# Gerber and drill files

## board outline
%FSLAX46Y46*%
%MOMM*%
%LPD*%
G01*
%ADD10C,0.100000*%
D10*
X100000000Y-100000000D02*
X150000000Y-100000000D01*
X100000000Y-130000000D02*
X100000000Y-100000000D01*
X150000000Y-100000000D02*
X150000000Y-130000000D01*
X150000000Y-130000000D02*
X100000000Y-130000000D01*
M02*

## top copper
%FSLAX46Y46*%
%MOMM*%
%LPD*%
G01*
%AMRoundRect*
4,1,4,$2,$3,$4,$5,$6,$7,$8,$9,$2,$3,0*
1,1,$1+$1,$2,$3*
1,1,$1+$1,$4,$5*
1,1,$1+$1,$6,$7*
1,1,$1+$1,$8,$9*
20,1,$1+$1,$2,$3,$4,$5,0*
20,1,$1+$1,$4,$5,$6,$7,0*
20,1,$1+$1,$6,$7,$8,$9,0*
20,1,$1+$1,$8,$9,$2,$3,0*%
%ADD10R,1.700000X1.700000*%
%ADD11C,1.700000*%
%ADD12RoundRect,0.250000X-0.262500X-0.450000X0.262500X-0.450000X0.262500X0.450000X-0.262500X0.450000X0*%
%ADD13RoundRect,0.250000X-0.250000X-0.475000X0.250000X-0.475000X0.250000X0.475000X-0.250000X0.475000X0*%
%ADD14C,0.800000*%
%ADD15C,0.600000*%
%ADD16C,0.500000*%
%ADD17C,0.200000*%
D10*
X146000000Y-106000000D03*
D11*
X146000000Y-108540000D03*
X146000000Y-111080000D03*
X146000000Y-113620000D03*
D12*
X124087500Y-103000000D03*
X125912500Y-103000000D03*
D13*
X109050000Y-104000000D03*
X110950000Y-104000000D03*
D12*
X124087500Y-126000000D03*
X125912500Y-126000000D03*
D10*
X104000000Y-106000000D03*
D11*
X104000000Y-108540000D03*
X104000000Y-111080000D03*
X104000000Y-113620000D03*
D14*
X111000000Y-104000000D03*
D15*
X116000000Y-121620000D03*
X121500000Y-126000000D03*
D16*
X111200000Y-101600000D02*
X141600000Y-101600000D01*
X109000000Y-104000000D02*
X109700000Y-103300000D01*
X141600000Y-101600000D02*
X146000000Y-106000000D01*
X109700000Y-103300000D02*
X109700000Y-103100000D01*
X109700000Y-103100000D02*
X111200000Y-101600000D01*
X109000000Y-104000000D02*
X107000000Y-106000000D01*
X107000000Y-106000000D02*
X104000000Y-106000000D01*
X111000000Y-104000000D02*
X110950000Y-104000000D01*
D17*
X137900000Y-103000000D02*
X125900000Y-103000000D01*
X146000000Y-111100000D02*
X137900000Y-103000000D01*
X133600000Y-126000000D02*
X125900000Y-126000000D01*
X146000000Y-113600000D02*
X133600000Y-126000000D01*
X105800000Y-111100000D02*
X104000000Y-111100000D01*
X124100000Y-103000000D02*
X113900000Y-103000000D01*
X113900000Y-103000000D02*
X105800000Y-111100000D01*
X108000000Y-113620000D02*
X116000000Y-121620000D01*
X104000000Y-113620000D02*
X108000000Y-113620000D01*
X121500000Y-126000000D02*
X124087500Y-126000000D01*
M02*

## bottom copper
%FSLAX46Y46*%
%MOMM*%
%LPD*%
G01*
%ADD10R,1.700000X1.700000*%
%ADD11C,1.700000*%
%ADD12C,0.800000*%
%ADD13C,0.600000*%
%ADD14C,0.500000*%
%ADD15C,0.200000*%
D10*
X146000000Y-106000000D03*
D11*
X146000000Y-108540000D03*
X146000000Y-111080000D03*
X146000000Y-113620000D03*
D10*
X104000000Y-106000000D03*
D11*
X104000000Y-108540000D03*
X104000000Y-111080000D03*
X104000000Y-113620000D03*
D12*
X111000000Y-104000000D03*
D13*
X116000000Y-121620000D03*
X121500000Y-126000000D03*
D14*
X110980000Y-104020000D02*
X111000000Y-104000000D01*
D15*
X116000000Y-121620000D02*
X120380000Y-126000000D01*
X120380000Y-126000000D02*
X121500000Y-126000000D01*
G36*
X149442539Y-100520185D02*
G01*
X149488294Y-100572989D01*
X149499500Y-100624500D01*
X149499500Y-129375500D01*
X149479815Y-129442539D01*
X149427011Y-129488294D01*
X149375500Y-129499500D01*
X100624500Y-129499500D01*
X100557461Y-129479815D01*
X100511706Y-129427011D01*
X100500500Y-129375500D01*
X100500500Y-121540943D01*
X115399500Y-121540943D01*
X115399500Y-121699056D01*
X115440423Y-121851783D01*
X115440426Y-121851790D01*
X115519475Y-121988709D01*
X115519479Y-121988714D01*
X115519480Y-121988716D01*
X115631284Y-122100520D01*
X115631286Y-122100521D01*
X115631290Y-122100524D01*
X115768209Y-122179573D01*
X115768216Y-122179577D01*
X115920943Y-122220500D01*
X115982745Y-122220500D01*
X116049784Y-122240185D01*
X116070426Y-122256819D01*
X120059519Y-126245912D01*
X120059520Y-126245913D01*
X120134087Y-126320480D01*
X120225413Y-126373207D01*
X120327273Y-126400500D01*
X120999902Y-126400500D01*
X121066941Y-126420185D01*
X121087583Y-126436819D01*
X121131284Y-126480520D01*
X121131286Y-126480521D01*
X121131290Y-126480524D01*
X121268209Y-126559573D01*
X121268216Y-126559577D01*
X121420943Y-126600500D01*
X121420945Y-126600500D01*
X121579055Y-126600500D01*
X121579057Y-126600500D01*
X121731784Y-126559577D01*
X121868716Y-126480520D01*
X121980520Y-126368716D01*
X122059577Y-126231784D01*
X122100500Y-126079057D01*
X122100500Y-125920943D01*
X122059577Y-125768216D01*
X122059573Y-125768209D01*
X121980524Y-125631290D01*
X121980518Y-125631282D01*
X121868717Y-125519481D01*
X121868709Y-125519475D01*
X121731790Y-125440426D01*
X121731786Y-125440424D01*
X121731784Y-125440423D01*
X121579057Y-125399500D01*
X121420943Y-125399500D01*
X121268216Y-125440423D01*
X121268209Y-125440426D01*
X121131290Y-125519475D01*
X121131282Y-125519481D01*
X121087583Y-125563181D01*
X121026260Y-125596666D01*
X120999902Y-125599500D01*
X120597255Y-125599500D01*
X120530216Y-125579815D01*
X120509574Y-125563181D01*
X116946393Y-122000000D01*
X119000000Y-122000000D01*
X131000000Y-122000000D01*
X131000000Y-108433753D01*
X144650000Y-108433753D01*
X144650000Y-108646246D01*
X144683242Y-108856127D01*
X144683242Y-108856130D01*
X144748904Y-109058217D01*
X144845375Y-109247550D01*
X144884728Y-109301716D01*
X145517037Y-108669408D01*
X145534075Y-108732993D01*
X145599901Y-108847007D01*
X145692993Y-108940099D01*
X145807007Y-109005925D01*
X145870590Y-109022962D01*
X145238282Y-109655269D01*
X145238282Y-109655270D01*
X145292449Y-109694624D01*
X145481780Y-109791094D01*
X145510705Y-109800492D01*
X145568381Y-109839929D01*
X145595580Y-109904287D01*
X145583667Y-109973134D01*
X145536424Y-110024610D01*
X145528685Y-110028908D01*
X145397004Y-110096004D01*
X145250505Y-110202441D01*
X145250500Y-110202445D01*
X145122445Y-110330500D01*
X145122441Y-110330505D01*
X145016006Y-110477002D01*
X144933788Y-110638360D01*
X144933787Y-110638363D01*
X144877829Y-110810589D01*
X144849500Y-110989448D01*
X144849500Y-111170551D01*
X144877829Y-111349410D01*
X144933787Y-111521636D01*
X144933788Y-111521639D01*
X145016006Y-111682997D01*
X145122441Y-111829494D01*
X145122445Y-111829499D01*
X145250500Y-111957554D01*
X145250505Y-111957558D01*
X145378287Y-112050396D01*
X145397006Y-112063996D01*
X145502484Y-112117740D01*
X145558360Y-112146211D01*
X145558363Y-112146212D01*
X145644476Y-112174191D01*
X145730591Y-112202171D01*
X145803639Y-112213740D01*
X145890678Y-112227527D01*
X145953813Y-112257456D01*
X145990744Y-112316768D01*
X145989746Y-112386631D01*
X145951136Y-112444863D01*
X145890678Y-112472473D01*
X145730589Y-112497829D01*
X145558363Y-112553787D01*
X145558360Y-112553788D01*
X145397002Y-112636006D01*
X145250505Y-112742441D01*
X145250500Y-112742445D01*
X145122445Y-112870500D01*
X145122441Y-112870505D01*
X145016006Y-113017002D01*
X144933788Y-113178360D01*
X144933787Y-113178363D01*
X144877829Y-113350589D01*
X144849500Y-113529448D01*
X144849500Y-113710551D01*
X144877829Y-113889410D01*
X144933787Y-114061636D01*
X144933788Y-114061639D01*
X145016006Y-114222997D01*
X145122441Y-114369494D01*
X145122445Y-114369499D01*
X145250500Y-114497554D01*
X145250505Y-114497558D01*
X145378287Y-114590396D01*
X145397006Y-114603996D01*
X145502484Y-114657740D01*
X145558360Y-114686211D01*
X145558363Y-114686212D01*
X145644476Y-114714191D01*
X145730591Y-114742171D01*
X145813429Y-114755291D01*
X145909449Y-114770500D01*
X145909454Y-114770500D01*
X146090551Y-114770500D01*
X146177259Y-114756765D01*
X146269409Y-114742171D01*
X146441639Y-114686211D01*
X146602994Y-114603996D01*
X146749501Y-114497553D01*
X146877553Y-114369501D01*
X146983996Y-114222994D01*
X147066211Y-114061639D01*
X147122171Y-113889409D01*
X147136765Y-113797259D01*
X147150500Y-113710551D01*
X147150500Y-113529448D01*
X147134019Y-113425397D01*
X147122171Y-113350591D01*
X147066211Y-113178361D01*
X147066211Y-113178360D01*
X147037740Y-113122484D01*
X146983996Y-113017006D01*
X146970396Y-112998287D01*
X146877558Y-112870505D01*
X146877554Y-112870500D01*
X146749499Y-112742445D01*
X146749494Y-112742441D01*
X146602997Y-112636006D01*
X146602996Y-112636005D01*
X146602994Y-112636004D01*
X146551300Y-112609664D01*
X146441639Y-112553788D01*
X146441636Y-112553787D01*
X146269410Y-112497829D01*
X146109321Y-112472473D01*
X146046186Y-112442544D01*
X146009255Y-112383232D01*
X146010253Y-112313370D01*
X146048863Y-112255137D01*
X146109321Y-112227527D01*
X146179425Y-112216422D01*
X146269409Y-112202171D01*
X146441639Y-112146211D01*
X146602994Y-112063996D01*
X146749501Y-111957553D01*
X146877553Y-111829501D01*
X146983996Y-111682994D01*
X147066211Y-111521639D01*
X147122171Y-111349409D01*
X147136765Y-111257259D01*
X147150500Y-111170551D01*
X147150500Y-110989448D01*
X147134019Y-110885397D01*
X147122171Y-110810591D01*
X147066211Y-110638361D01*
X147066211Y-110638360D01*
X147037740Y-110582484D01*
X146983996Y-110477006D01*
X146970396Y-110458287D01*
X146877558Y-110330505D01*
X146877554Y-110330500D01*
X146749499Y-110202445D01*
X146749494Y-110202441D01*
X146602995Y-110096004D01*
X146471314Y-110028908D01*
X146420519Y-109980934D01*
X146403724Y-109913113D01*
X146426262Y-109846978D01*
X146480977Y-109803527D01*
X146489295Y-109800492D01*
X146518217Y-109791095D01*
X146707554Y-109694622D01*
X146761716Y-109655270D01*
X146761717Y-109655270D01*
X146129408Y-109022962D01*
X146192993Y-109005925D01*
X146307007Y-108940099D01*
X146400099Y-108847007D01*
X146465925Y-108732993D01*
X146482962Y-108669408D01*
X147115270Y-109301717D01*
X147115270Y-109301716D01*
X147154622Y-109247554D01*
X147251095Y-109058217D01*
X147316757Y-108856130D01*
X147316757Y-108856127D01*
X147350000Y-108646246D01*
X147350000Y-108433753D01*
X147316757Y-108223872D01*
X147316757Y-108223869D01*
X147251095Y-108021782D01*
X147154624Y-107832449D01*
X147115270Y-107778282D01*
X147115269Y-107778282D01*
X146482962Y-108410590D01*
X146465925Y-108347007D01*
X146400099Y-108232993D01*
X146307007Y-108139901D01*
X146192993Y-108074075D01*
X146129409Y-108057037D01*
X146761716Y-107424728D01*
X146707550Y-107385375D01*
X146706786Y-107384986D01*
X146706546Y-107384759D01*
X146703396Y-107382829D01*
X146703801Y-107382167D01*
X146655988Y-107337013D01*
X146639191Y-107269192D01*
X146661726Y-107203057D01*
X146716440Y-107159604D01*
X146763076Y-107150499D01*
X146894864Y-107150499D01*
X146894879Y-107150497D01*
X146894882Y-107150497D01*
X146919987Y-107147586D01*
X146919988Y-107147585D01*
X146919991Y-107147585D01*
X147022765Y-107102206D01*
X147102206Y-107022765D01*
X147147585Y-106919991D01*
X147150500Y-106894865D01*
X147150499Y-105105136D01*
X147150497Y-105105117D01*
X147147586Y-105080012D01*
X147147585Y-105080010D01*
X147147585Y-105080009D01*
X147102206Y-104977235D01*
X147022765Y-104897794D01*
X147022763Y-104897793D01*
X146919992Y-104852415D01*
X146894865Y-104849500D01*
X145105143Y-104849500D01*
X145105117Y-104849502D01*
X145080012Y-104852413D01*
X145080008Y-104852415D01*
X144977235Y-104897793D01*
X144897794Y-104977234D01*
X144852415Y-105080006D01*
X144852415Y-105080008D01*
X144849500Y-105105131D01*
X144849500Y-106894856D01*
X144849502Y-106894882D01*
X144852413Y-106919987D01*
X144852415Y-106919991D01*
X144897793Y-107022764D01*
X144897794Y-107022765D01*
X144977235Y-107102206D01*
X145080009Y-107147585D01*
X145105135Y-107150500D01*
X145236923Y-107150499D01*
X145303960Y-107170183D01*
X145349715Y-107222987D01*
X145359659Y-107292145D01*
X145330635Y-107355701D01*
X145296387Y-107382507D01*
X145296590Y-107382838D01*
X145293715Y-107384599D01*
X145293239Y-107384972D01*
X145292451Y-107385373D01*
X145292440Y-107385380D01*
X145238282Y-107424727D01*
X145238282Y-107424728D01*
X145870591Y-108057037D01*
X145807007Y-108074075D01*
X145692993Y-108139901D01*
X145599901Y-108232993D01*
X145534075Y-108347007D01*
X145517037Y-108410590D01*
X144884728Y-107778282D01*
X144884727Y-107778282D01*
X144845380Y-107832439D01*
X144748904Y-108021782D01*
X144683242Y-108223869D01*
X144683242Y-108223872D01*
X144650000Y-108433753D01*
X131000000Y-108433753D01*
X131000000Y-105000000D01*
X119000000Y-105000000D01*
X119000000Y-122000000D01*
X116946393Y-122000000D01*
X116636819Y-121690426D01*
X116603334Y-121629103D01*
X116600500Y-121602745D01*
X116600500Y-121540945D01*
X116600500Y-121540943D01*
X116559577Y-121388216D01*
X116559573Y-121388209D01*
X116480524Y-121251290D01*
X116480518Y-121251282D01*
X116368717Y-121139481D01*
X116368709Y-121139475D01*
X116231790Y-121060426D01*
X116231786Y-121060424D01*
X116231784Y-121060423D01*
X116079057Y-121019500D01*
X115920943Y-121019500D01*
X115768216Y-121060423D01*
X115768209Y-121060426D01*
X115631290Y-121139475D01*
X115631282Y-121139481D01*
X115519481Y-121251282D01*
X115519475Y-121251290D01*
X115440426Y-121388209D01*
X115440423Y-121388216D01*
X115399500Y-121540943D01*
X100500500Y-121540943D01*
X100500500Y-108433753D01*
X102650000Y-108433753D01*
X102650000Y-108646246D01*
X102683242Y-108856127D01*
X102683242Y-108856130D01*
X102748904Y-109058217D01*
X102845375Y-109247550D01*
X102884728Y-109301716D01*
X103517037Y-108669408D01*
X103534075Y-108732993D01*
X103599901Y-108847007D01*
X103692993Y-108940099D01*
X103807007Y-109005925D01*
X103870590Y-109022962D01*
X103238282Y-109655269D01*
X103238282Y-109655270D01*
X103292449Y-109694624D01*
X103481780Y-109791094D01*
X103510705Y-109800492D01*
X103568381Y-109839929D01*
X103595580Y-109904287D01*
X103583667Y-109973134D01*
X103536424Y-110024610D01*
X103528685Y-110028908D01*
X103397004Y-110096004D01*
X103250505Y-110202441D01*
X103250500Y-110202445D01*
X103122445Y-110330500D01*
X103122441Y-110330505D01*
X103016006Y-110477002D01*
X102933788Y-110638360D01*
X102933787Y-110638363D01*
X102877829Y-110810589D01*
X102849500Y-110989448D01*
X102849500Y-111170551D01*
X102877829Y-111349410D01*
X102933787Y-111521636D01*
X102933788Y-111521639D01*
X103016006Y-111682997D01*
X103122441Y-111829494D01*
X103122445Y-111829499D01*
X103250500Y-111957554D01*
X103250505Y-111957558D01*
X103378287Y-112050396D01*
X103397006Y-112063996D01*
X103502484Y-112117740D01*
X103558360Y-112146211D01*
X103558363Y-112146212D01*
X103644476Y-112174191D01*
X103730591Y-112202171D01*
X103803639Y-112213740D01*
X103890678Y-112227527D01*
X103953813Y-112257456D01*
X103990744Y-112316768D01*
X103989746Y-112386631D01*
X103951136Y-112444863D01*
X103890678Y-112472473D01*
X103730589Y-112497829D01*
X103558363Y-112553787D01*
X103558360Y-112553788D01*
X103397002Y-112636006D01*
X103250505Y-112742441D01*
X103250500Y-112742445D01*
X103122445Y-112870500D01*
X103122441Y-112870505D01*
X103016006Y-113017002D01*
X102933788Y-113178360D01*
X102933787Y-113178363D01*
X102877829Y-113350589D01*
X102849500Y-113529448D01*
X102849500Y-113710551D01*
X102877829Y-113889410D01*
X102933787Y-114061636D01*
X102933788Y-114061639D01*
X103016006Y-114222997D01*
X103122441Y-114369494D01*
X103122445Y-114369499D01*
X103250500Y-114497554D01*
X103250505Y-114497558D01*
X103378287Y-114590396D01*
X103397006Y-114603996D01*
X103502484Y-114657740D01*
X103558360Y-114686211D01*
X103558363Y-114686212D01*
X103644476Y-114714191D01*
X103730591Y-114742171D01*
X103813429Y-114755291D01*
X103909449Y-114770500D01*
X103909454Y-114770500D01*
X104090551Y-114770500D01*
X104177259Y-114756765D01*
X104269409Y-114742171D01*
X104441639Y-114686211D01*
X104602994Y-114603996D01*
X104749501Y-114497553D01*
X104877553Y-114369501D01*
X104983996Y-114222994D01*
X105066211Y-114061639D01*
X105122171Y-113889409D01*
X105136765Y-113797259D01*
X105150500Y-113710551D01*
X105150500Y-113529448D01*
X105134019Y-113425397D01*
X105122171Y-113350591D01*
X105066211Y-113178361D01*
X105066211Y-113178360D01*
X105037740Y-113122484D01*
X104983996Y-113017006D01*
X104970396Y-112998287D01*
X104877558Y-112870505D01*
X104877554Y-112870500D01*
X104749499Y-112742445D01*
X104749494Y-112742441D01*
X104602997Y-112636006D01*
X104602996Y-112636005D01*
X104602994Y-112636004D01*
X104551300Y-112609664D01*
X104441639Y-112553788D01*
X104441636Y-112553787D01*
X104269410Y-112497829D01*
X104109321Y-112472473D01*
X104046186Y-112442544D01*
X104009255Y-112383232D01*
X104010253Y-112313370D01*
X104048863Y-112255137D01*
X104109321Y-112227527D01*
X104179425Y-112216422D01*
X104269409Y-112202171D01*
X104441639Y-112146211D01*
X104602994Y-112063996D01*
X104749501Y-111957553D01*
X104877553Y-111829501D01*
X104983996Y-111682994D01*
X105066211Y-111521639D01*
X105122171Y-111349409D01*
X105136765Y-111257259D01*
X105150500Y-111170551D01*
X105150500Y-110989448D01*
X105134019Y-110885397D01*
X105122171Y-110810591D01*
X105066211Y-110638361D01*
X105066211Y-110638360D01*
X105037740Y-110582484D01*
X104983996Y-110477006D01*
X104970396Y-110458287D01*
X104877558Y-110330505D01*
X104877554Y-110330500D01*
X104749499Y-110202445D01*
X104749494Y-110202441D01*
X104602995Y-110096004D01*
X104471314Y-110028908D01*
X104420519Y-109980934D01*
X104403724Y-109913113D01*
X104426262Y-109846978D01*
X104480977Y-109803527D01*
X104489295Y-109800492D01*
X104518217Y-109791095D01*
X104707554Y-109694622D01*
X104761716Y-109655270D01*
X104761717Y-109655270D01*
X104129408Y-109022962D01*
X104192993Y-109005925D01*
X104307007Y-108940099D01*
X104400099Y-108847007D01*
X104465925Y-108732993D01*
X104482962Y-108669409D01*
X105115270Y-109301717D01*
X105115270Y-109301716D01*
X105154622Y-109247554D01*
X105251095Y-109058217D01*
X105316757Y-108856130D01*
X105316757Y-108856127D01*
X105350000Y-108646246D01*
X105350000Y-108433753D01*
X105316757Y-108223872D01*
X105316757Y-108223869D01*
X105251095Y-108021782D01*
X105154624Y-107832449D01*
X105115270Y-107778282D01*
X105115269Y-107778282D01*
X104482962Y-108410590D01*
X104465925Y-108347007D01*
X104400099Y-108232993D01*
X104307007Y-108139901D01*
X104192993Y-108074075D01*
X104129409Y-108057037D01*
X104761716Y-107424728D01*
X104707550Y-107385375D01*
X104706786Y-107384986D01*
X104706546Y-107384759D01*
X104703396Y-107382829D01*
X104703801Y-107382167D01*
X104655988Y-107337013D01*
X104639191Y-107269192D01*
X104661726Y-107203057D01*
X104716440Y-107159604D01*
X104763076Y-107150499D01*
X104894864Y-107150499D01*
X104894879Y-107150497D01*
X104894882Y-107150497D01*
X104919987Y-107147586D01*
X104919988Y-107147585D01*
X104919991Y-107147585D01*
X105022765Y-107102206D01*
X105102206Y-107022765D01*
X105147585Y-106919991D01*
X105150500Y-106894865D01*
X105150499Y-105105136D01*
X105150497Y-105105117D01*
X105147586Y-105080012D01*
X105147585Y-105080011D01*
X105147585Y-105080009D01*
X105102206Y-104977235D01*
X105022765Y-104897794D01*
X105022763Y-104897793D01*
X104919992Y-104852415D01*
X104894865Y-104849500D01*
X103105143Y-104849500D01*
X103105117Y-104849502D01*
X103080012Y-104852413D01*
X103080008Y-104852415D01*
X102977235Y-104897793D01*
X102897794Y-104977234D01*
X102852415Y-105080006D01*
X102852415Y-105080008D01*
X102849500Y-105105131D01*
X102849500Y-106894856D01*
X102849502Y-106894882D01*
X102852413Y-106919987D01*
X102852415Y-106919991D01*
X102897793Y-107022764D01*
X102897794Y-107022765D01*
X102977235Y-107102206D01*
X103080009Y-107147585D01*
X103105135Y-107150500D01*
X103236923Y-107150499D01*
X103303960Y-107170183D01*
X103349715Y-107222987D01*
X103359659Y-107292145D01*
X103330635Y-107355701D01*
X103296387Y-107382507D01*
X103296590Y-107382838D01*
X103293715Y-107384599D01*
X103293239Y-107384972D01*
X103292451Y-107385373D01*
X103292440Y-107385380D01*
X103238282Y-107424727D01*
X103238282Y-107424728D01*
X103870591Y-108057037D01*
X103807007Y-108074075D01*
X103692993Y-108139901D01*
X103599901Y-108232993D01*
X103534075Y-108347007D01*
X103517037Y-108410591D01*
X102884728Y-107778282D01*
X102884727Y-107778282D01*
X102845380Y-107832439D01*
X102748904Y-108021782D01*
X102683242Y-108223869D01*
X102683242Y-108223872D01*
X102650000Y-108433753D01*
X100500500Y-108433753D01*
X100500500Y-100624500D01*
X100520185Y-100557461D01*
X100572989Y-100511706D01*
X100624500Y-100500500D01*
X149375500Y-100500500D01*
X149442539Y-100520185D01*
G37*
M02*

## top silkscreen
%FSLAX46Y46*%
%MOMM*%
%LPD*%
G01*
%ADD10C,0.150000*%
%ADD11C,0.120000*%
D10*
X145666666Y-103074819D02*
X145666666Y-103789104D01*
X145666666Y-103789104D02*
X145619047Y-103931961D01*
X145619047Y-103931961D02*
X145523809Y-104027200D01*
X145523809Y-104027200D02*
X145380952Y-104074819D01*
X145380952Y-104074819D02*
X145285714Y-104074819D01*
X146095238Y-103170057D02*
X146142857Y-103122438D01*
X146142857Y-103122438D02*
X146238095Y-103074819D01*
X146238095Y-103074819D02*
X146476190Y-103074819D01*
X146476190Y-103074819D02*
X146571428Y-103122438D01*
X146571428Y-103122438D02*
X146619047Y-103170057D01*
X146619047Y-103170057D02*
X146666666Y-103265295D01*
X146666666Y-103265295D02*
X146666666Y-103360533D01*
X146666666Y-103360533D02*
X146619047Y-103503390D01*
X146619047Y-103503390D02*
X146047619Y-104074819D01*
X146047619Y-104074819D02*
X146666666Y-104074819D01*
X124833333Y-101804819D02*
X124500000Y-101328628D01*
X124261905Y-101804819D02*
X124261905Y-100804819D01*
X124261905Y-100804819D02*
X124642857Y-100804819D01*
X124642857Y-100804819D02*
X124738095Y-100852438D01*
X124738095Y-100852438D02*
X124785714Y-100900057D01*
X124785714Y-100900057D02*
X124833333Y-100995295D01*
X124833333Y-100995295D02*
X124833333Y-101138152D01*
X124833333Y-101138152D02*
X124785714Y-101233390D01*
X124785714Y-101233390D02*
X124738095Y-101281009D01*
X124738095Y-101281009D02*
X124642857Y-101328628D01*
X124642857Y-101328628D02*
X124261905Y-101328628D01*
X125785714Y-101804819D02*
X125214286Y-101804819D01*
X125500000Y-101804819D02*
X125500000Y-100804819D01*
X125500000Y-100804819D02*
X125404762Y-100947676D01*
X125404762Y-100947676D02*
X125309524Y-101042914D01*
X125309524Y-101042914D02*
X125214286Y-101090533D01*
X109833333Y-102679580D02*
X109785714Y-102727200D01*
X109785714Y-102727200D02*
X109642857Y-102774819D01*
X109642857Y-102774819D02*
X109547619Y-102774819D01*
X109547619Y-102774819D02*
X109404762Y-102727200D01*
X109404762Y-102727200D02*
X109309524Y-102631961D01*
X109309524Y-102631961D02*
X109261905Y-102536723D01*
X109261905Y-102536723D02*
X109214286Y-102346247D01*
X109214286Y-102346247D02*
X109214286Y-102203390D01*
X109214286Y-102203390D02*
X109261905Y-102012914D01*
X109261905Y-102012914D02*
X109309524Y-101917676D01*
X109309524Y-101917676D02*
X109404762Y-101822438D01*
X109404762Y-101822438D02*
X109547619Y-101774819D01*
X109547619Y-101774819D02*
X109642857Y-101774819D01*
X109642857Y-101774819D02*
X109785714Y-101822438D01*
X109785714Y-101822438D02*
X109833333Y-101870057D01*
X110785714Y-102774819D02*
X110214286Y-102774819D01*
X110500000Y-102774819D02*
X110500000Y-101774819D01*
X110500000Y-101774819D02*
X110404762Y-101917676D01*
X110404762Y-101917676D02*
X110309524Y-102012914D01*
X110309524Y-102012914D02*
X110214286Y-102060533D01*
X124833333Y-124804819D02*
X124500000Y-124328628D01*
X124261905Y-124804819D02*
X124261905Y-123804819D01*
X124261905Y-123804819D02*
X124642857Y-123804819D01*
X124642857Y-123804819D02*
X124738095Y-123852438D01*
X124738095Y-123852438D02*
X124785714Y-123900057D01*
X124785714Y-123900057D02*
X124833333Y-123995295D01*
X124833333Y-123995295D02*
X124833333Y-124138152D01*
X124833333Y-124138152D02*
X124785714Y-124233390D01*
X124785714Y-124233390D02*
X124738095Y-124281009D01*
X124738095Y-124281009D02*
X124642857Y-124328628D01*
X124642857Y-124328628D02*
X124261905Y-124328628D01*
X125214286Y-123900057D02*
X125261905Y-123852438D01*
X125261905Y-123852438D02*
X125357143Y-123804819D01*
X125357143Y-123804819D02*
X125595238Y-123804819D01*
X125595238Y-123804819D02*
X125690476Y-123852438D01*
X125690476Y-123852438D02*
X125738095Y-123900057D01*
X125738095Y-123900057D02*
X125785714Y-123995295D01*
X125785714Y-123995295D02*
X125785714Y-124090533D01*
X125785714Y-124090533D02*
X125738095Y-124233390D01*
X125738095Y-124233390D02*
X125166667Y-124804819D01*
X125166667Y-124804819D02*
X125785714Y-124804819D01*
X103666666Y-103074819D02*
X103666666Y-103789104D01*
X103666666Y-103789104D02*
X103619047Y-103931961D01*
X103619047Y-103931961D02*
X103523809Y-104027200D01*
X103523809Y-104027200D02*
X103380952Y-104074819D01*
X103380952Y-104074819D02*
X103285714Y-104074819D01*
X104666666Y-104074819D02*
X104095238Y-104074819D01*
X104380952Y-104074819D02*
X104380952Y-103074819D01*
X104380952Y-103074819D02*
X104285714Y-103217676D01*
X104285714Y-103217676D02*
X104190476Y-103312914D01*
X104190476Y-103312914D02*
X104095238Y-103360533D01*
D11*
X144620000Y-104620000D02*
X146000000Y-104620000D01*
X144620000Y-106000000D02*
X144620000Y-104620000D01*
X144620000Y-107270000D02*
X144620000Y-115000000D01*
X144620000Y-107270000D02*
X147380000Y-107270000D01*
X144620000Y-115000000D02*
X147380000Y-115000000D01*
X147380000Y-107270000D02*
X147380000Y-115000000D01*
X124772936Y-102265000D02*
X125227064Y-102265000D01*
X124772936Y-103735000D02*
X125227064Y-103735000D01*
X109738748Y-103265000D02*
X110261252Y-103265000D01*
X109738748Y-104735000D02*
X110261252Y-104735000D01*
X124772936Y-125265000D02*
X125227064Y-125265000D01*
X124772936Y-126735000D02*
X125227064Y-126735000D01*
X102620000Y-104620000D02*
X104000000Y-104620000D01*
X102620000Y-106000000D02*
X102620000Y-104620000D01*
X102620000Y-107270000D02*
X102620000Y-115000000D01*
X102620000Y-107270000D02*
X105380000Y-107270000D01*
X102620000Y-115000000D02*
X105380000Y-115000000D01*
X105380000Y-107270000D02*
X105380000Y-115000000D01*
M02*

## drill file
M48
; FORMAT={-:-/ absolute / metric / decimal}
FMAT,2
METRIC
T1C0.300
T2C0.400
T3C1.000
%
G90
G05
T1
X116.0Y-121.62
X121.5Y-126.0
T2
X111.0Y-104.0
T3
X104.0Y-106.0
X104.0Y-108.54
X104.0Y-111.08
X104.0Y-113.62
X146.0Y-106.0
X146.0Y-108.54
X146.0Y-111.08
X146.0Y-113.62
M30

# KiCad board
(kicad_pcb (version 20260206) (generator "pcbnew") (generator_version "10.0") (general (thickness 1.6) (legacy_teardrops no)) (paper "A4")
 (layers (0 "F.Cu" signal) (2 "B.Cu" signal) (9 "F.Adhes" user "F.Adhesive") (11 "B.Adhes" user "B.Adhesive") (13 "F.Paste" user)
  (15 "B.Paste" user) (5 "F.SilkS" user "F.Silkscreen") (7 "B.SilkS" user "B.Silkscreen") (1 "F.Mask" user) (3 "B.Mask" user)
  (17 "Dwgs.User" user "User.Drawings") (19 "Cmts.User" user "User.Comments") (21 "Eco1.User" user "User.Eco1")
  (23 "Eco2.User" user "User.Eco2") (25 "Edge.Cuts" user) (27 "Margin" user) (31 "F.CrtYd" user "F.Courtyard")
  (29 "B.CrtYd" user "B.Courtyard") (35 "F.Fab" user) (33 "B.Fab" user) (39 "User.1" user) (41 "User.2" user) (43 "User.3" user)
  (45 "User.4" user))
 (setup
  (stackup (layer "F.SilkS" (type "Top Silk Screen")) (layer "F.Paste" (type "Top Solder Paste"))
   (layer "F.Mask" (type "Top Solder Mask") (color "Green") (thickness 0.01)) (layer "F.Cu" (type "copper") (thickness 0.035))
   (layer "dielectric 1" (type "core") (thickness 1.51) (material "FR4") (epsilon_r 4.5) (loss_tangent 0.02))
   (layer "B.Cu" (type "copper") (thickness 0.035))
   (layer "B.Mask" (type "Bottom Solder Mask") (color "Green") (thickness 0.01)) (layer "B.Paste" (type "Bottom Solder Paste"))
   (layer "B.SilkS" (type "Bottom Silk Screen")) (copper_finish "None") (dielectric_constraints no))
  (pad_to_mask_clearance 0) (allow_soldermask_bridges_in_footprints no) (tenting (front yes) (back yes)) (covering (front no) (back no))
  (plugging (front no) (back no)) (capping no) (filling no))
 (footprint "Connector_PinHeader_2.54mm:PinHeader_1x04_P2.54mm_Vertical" (layer "F.Cu") (at 146 106)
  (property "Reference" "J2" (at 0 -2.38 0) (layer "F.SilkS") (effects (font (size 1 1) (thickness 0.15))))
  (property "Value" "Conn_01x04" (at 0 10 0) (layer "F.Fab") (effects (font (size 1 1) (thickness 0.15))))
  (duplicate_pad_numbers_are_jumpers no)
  (fp_line (start -1.38 -1.38) (end 0 -1.38) (stroke (width 0.12) (type solid)) (layer "F.SilkS"))
  (fp_line (start -1.38 0) (end -1.38 -1.38) (stroke (width 0.12) (type solid)) (layer "F.SilkS"))
  (fp_line (start -1.38 1.27) (end -1.38 9) (stroke (width 0.12) (type solid)) (layer "F.SilkS"))
  (fp_line (start -1.38 1.27) (end 1.38 1.27) (stroke (width 0.12) (type solid)) (layer "F.SilkS"))
  (fp_line (start -1.38 9) (end 1.38 9) (stroke (width 0.12) (type solid)) (layer "F.SilkS"))
  (fp_line (start 1.38 1.27) (end 1.38 9) (stroke (width 0.12) (type solid)) (layer "F.SilkS"))
  (pad "1" thru_hole rect (at 0 0) (size 1.7 1.7) (drill 1) (layers "*.Cu" "*.Mask") (remove_unused_layers no) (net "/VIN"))
  (pad "2" thru_hole circle (at 0 2.54) (size 1.7 1.7) (drill 1) (layers "*.Cu" "*.Mask") (remove_unused_layers no) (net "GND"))
  (pad "3" thru_hole circle (at 0 5.08) (size 1.7 1.7) (drill 1) (layers "*.Cu" "*.Mask") (remove_unused_layers no) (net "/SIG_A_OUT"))
  (pad "4" thru_hole circle (at 0 7.62) (size 1.7 1.7) (drill 1) (layers "*.Cu" "*.Mask") (remove_unused_layers no) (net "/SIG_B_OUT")))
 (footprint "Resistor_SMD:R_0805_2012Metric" (layer "F.Cu") (at 125 103)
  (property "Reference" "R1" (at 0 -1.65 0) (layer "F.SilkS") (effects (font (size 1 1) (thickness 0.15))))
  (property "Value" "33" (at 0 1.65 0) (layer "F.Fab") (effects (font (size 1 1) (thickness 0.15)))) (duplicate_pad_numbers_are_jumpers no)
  (fp_line (start -0.227064 -0.735) (end 0.227064 -0.735) (stroke (width 0.12) (type solid)) (layer "F.SilkS"))
  (fp_line (start -0.227064 0.735) (end 0.227064 0.735) (stroke (width 0.12) (type solid)) (layer "F.SilkS"))
  (pad "1" smd roundrect (at -0.9125 0) (size 1.025 1.4) (layers "F.Cu" "F.Mask" "F.Paste") (roundrect_rratio 0.243902) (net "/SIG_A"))
  (pad "2" smd roundrect (at 0.9125 0) (size 1.025 1.4) (layers "F.Cu" "F.Mask" "F.Paste") (roundrect_rratio 0.243902) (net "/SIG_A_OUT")))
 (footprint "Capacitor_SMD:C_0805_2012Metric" (layer "F.Cu") (at 110 104)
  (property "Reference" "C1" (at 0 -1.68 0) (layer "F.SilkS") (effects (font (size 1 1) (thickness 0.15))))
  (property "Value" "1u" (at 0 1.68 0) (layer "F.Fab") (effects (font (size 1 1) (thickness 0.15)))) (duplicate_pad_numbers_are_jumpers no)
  (fp_line (start -0.261252 -0.735) (end 0.261252 -0.735) (stroke (width 0.12) (type solid)) (layer "F.SilkS"))
  (fp_line (start -0.261252 0.735) (end 0.261252 0.735) (stroke (width 0.12) (type solid)) (layer "F.SilkS"))
  (pad "1" smd roundrect (at -0.95 0) (size 1 1.45) (layers "F.Cu" "F.Mask" "F.Paste") (roundrect_rratio 0.25) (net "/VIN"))
  (pad "2" smd roundrect (at 0.95 0) (size 1 1.45) (layers "F.Cu" "F.Mask" "F.Paste") (roundrect_rratio 0.25) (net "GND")))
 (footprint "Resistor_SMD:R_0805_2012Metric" (layer "F.Cu") (at 125 126)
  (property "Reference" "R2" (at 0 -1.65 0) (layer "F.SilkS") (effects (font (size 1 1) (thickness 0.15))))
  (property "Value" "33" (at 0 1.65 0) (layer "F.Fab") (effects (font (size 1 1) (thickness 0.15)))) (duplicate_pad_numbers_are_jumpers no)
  (fp_line (start -0.227064 -0.735) (end 0.227064 -0.735) (stroke (width 0.12) (type solid)) (layer "F.SilkS"))
  (fp_line (start -0.227064 0.735) (end 0.227064 0.735) (stroke (width 0.12) (type solid)) (layer "F.SilkS"))
  (pad "1" smd roundrect (at -0.9125 0) (size 1.025 1.4) (layers "F.Cu" "F.Mask" "F.Paste") (roundrect_rratio 0.243902) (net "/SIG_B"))
  (pad "2" smd roundrect (at 0.9125 0) (size 1.025 1.4) (layers "F.Cu" "F.Mask" "F.Paste") (roundrect_rratio 0.243902) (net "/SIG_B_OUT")))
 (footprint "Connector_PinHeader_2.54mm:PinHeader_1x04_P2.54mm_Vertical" (layer "F.Cu") (at 104 106)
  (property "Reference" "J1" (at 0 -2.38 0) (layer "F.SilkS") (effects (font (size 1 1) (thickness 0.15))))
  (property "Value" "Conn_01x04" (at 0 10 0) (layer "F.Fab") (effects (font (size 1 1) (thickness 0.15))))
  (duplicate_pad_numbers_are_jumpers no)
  (fp_line (start -1.38 -1.38) (end 0 -1.38) (stroke (width 0.12) (type solid)) (layer "F.SilkS"))
  (fp_line (start -1.38 0) (end -1.38 -1.38) (stroke (width 0.12) (type solid)) (layer "F.SilkS"))
  (fp_line (start -1.38 1.27) (end -1.38 9) (stroke (width 0.12) (type solid)) (layer "F.SilkS"))
  (fp_line (start -1.38 1.27) (end 1.38 1.27) (stroke (width 0.12) (type solid)) (layer "F.SilkS"))
  (fp_line (start -1.38 9) (end 1.38 9) (stroke (width 0.12) (type solid)) (layer "F.SilkS"))
  (fp_line (start 1.38 1.27) (end 1.38 9) (stroke (width 0.12) (type solid)) (layer "F.SilkS"))
  (pad "1" thru_hole rect (at 0 0) (size 1.7 1.7) (drill 1) (layers "*.Cu" "*.Mask") (remove_unused_layers no) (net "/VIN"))
  (pad "2" thru_hole circle (at 0 2.54) (size 1.7 1.7) (drill 1) (layers "*.Cu" "*.Mask") (remove_unused_layers no) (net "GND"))
  (pad "3" thru_hole circle (at 0 5.08) (size 1.7 1.7) (drill 1) (layers "*.Cu" "*.Mask") (remove_unused_layers no) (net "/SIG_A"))
  (pad "4" thru_hole circle (at 0 7.62) (size 1.7 1.7) (drill 1) (layers "*.Cu" "*.Mask") (remove_unused_layers no) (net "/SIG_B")))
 (gr_line (start 100 100) (end 150 100) (stroke (width 0.1) (type default)) (layer "Edge.Cuts"))
 (gr_line (start 100 130) (end 100 100) (stroke (width 0.1) (type default)) (layer "Edge.Cuts"))
 (gr_line (start 150 100) (end 150 130) (stroke (width 0.1) (type default)) (layer "Edge.Cuts"))
 (gr_line (start 150 130) (end 100 130) (stroke (width 0.1) (type default)) (layer "Edge.Cuts"))
 (segment (start 111.2 101.6) (end 141.6 101.6) (width 0.5) (layer "F.Cu") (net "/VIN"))
 (segment (start 109 104) (end 109.7 103.3) (width 0.5) (layer "F.Cu") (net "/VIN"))
 (segment (start 141.6 101.6) (end 146 106) (width 0.5) (layer "F.Cu") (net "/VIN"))
 (segment (start 109.7 103.3) (end 109.7 103.1) (width 0.5) (layer "F.Cu") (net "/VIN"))
 (segment (start 109.7 103.1) (end 111.2 101.6) (width 0.5) (layer "F.Cu") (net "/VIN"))
 (segment (start 109 104) (end 107 106) (width 0.5) (layer "F.Cu") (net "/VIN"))
 (segment (start 107 106) (end 104 106) (width 0.5) (layer "F.Cu") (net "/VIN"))
 (segment (start 111 104) (end 110.95 104) (width 0.5) (layer "F.Cu") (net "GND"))
 (via (at 111 104) (size 0.8) (drill 0.4) (layers "F.Cu" "B.Cu") (capping yes) (filling yes) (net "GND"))
 (segment (start 110.98 104.02) (end 111 104) (width 0.5) (layer "B.Cu") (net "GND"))
 (segment (start 137.9 103) (end 125.9 103) (width 0.2) (layer "F.Cu") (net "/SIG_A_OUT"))
 (segment (start 146 111.1) (end 137.9 103) (width 0.2) (layer "F.Cu") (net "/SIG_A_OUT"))
 (segment (start 133.6 126) (end 125.9 126) (width 0.2) (layer "F.Cu") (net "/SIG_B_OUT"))
 (segment (start 146 113.6) (end 133.6 126) (width 0.2) (layer "F.Cu") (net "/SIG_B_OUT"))
 (segment (start 105.8 111.1) (end 104 111.1) (width 0.2) (layer "F.Cu") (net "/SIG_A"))
 (segment (start 124.1 103) (end 113.9 103) (width 0.2) (layer "F.Cu") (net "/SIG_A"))
 (segment (start 113.9 103) (end 105.8 111.1) (width 0.2) (layer "F.Cu") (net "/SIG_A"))
 (segment (start 108 113.62) (end 116 121.62) (width 0.2) (locked yes) (layer "F.Cu") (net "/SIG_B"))
 (segment (start 104 113.62) (end 108 113.62) (width 0.2) (locked yes) (layer "F.Cu") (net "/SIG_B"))
 (segment (start 121.5 126) (end 124.0875 126) (width 0.2) (locked yes) (layer "F.Cu") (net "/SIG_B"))
 (via (at 116 121.62) (size 0.6) (drill 0.3) (layers "F.Cu" "B.Cu") (locked yes) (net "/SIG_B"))
 (via (at 121.5 126) (size 0.6) (drill 0.3) (layers "F.Cu" "B.Cu") (locked yes) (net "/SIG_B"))
 (segment (start 116 121.62) (end 120.38 126) (width 0.2) (locked yes) (layer "B.Cu") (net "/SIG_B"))
 (segment (start 120.38 126) (end 121.5 126) (width 0.2) (locked yes) (layer "B.Cu") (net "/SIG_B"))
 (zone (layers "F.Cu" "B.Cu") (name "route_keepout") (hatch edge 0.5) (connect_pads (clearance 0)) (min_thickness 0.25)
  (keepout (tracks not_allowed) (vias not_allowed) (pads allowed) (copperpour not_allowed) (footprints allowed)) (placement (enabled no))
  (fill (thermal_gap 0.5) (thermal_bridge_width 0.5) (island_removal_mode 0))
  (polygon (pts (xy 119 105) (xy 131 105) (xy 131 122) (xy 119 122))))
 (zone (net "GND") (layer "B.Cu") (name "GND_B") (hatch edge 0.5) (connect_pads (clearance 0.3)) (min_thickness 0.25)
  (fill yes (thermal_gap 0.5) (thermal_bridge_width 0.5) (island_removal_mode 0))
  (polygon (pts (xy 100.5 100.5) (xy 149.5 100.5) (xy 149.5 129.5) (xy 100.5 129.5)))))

